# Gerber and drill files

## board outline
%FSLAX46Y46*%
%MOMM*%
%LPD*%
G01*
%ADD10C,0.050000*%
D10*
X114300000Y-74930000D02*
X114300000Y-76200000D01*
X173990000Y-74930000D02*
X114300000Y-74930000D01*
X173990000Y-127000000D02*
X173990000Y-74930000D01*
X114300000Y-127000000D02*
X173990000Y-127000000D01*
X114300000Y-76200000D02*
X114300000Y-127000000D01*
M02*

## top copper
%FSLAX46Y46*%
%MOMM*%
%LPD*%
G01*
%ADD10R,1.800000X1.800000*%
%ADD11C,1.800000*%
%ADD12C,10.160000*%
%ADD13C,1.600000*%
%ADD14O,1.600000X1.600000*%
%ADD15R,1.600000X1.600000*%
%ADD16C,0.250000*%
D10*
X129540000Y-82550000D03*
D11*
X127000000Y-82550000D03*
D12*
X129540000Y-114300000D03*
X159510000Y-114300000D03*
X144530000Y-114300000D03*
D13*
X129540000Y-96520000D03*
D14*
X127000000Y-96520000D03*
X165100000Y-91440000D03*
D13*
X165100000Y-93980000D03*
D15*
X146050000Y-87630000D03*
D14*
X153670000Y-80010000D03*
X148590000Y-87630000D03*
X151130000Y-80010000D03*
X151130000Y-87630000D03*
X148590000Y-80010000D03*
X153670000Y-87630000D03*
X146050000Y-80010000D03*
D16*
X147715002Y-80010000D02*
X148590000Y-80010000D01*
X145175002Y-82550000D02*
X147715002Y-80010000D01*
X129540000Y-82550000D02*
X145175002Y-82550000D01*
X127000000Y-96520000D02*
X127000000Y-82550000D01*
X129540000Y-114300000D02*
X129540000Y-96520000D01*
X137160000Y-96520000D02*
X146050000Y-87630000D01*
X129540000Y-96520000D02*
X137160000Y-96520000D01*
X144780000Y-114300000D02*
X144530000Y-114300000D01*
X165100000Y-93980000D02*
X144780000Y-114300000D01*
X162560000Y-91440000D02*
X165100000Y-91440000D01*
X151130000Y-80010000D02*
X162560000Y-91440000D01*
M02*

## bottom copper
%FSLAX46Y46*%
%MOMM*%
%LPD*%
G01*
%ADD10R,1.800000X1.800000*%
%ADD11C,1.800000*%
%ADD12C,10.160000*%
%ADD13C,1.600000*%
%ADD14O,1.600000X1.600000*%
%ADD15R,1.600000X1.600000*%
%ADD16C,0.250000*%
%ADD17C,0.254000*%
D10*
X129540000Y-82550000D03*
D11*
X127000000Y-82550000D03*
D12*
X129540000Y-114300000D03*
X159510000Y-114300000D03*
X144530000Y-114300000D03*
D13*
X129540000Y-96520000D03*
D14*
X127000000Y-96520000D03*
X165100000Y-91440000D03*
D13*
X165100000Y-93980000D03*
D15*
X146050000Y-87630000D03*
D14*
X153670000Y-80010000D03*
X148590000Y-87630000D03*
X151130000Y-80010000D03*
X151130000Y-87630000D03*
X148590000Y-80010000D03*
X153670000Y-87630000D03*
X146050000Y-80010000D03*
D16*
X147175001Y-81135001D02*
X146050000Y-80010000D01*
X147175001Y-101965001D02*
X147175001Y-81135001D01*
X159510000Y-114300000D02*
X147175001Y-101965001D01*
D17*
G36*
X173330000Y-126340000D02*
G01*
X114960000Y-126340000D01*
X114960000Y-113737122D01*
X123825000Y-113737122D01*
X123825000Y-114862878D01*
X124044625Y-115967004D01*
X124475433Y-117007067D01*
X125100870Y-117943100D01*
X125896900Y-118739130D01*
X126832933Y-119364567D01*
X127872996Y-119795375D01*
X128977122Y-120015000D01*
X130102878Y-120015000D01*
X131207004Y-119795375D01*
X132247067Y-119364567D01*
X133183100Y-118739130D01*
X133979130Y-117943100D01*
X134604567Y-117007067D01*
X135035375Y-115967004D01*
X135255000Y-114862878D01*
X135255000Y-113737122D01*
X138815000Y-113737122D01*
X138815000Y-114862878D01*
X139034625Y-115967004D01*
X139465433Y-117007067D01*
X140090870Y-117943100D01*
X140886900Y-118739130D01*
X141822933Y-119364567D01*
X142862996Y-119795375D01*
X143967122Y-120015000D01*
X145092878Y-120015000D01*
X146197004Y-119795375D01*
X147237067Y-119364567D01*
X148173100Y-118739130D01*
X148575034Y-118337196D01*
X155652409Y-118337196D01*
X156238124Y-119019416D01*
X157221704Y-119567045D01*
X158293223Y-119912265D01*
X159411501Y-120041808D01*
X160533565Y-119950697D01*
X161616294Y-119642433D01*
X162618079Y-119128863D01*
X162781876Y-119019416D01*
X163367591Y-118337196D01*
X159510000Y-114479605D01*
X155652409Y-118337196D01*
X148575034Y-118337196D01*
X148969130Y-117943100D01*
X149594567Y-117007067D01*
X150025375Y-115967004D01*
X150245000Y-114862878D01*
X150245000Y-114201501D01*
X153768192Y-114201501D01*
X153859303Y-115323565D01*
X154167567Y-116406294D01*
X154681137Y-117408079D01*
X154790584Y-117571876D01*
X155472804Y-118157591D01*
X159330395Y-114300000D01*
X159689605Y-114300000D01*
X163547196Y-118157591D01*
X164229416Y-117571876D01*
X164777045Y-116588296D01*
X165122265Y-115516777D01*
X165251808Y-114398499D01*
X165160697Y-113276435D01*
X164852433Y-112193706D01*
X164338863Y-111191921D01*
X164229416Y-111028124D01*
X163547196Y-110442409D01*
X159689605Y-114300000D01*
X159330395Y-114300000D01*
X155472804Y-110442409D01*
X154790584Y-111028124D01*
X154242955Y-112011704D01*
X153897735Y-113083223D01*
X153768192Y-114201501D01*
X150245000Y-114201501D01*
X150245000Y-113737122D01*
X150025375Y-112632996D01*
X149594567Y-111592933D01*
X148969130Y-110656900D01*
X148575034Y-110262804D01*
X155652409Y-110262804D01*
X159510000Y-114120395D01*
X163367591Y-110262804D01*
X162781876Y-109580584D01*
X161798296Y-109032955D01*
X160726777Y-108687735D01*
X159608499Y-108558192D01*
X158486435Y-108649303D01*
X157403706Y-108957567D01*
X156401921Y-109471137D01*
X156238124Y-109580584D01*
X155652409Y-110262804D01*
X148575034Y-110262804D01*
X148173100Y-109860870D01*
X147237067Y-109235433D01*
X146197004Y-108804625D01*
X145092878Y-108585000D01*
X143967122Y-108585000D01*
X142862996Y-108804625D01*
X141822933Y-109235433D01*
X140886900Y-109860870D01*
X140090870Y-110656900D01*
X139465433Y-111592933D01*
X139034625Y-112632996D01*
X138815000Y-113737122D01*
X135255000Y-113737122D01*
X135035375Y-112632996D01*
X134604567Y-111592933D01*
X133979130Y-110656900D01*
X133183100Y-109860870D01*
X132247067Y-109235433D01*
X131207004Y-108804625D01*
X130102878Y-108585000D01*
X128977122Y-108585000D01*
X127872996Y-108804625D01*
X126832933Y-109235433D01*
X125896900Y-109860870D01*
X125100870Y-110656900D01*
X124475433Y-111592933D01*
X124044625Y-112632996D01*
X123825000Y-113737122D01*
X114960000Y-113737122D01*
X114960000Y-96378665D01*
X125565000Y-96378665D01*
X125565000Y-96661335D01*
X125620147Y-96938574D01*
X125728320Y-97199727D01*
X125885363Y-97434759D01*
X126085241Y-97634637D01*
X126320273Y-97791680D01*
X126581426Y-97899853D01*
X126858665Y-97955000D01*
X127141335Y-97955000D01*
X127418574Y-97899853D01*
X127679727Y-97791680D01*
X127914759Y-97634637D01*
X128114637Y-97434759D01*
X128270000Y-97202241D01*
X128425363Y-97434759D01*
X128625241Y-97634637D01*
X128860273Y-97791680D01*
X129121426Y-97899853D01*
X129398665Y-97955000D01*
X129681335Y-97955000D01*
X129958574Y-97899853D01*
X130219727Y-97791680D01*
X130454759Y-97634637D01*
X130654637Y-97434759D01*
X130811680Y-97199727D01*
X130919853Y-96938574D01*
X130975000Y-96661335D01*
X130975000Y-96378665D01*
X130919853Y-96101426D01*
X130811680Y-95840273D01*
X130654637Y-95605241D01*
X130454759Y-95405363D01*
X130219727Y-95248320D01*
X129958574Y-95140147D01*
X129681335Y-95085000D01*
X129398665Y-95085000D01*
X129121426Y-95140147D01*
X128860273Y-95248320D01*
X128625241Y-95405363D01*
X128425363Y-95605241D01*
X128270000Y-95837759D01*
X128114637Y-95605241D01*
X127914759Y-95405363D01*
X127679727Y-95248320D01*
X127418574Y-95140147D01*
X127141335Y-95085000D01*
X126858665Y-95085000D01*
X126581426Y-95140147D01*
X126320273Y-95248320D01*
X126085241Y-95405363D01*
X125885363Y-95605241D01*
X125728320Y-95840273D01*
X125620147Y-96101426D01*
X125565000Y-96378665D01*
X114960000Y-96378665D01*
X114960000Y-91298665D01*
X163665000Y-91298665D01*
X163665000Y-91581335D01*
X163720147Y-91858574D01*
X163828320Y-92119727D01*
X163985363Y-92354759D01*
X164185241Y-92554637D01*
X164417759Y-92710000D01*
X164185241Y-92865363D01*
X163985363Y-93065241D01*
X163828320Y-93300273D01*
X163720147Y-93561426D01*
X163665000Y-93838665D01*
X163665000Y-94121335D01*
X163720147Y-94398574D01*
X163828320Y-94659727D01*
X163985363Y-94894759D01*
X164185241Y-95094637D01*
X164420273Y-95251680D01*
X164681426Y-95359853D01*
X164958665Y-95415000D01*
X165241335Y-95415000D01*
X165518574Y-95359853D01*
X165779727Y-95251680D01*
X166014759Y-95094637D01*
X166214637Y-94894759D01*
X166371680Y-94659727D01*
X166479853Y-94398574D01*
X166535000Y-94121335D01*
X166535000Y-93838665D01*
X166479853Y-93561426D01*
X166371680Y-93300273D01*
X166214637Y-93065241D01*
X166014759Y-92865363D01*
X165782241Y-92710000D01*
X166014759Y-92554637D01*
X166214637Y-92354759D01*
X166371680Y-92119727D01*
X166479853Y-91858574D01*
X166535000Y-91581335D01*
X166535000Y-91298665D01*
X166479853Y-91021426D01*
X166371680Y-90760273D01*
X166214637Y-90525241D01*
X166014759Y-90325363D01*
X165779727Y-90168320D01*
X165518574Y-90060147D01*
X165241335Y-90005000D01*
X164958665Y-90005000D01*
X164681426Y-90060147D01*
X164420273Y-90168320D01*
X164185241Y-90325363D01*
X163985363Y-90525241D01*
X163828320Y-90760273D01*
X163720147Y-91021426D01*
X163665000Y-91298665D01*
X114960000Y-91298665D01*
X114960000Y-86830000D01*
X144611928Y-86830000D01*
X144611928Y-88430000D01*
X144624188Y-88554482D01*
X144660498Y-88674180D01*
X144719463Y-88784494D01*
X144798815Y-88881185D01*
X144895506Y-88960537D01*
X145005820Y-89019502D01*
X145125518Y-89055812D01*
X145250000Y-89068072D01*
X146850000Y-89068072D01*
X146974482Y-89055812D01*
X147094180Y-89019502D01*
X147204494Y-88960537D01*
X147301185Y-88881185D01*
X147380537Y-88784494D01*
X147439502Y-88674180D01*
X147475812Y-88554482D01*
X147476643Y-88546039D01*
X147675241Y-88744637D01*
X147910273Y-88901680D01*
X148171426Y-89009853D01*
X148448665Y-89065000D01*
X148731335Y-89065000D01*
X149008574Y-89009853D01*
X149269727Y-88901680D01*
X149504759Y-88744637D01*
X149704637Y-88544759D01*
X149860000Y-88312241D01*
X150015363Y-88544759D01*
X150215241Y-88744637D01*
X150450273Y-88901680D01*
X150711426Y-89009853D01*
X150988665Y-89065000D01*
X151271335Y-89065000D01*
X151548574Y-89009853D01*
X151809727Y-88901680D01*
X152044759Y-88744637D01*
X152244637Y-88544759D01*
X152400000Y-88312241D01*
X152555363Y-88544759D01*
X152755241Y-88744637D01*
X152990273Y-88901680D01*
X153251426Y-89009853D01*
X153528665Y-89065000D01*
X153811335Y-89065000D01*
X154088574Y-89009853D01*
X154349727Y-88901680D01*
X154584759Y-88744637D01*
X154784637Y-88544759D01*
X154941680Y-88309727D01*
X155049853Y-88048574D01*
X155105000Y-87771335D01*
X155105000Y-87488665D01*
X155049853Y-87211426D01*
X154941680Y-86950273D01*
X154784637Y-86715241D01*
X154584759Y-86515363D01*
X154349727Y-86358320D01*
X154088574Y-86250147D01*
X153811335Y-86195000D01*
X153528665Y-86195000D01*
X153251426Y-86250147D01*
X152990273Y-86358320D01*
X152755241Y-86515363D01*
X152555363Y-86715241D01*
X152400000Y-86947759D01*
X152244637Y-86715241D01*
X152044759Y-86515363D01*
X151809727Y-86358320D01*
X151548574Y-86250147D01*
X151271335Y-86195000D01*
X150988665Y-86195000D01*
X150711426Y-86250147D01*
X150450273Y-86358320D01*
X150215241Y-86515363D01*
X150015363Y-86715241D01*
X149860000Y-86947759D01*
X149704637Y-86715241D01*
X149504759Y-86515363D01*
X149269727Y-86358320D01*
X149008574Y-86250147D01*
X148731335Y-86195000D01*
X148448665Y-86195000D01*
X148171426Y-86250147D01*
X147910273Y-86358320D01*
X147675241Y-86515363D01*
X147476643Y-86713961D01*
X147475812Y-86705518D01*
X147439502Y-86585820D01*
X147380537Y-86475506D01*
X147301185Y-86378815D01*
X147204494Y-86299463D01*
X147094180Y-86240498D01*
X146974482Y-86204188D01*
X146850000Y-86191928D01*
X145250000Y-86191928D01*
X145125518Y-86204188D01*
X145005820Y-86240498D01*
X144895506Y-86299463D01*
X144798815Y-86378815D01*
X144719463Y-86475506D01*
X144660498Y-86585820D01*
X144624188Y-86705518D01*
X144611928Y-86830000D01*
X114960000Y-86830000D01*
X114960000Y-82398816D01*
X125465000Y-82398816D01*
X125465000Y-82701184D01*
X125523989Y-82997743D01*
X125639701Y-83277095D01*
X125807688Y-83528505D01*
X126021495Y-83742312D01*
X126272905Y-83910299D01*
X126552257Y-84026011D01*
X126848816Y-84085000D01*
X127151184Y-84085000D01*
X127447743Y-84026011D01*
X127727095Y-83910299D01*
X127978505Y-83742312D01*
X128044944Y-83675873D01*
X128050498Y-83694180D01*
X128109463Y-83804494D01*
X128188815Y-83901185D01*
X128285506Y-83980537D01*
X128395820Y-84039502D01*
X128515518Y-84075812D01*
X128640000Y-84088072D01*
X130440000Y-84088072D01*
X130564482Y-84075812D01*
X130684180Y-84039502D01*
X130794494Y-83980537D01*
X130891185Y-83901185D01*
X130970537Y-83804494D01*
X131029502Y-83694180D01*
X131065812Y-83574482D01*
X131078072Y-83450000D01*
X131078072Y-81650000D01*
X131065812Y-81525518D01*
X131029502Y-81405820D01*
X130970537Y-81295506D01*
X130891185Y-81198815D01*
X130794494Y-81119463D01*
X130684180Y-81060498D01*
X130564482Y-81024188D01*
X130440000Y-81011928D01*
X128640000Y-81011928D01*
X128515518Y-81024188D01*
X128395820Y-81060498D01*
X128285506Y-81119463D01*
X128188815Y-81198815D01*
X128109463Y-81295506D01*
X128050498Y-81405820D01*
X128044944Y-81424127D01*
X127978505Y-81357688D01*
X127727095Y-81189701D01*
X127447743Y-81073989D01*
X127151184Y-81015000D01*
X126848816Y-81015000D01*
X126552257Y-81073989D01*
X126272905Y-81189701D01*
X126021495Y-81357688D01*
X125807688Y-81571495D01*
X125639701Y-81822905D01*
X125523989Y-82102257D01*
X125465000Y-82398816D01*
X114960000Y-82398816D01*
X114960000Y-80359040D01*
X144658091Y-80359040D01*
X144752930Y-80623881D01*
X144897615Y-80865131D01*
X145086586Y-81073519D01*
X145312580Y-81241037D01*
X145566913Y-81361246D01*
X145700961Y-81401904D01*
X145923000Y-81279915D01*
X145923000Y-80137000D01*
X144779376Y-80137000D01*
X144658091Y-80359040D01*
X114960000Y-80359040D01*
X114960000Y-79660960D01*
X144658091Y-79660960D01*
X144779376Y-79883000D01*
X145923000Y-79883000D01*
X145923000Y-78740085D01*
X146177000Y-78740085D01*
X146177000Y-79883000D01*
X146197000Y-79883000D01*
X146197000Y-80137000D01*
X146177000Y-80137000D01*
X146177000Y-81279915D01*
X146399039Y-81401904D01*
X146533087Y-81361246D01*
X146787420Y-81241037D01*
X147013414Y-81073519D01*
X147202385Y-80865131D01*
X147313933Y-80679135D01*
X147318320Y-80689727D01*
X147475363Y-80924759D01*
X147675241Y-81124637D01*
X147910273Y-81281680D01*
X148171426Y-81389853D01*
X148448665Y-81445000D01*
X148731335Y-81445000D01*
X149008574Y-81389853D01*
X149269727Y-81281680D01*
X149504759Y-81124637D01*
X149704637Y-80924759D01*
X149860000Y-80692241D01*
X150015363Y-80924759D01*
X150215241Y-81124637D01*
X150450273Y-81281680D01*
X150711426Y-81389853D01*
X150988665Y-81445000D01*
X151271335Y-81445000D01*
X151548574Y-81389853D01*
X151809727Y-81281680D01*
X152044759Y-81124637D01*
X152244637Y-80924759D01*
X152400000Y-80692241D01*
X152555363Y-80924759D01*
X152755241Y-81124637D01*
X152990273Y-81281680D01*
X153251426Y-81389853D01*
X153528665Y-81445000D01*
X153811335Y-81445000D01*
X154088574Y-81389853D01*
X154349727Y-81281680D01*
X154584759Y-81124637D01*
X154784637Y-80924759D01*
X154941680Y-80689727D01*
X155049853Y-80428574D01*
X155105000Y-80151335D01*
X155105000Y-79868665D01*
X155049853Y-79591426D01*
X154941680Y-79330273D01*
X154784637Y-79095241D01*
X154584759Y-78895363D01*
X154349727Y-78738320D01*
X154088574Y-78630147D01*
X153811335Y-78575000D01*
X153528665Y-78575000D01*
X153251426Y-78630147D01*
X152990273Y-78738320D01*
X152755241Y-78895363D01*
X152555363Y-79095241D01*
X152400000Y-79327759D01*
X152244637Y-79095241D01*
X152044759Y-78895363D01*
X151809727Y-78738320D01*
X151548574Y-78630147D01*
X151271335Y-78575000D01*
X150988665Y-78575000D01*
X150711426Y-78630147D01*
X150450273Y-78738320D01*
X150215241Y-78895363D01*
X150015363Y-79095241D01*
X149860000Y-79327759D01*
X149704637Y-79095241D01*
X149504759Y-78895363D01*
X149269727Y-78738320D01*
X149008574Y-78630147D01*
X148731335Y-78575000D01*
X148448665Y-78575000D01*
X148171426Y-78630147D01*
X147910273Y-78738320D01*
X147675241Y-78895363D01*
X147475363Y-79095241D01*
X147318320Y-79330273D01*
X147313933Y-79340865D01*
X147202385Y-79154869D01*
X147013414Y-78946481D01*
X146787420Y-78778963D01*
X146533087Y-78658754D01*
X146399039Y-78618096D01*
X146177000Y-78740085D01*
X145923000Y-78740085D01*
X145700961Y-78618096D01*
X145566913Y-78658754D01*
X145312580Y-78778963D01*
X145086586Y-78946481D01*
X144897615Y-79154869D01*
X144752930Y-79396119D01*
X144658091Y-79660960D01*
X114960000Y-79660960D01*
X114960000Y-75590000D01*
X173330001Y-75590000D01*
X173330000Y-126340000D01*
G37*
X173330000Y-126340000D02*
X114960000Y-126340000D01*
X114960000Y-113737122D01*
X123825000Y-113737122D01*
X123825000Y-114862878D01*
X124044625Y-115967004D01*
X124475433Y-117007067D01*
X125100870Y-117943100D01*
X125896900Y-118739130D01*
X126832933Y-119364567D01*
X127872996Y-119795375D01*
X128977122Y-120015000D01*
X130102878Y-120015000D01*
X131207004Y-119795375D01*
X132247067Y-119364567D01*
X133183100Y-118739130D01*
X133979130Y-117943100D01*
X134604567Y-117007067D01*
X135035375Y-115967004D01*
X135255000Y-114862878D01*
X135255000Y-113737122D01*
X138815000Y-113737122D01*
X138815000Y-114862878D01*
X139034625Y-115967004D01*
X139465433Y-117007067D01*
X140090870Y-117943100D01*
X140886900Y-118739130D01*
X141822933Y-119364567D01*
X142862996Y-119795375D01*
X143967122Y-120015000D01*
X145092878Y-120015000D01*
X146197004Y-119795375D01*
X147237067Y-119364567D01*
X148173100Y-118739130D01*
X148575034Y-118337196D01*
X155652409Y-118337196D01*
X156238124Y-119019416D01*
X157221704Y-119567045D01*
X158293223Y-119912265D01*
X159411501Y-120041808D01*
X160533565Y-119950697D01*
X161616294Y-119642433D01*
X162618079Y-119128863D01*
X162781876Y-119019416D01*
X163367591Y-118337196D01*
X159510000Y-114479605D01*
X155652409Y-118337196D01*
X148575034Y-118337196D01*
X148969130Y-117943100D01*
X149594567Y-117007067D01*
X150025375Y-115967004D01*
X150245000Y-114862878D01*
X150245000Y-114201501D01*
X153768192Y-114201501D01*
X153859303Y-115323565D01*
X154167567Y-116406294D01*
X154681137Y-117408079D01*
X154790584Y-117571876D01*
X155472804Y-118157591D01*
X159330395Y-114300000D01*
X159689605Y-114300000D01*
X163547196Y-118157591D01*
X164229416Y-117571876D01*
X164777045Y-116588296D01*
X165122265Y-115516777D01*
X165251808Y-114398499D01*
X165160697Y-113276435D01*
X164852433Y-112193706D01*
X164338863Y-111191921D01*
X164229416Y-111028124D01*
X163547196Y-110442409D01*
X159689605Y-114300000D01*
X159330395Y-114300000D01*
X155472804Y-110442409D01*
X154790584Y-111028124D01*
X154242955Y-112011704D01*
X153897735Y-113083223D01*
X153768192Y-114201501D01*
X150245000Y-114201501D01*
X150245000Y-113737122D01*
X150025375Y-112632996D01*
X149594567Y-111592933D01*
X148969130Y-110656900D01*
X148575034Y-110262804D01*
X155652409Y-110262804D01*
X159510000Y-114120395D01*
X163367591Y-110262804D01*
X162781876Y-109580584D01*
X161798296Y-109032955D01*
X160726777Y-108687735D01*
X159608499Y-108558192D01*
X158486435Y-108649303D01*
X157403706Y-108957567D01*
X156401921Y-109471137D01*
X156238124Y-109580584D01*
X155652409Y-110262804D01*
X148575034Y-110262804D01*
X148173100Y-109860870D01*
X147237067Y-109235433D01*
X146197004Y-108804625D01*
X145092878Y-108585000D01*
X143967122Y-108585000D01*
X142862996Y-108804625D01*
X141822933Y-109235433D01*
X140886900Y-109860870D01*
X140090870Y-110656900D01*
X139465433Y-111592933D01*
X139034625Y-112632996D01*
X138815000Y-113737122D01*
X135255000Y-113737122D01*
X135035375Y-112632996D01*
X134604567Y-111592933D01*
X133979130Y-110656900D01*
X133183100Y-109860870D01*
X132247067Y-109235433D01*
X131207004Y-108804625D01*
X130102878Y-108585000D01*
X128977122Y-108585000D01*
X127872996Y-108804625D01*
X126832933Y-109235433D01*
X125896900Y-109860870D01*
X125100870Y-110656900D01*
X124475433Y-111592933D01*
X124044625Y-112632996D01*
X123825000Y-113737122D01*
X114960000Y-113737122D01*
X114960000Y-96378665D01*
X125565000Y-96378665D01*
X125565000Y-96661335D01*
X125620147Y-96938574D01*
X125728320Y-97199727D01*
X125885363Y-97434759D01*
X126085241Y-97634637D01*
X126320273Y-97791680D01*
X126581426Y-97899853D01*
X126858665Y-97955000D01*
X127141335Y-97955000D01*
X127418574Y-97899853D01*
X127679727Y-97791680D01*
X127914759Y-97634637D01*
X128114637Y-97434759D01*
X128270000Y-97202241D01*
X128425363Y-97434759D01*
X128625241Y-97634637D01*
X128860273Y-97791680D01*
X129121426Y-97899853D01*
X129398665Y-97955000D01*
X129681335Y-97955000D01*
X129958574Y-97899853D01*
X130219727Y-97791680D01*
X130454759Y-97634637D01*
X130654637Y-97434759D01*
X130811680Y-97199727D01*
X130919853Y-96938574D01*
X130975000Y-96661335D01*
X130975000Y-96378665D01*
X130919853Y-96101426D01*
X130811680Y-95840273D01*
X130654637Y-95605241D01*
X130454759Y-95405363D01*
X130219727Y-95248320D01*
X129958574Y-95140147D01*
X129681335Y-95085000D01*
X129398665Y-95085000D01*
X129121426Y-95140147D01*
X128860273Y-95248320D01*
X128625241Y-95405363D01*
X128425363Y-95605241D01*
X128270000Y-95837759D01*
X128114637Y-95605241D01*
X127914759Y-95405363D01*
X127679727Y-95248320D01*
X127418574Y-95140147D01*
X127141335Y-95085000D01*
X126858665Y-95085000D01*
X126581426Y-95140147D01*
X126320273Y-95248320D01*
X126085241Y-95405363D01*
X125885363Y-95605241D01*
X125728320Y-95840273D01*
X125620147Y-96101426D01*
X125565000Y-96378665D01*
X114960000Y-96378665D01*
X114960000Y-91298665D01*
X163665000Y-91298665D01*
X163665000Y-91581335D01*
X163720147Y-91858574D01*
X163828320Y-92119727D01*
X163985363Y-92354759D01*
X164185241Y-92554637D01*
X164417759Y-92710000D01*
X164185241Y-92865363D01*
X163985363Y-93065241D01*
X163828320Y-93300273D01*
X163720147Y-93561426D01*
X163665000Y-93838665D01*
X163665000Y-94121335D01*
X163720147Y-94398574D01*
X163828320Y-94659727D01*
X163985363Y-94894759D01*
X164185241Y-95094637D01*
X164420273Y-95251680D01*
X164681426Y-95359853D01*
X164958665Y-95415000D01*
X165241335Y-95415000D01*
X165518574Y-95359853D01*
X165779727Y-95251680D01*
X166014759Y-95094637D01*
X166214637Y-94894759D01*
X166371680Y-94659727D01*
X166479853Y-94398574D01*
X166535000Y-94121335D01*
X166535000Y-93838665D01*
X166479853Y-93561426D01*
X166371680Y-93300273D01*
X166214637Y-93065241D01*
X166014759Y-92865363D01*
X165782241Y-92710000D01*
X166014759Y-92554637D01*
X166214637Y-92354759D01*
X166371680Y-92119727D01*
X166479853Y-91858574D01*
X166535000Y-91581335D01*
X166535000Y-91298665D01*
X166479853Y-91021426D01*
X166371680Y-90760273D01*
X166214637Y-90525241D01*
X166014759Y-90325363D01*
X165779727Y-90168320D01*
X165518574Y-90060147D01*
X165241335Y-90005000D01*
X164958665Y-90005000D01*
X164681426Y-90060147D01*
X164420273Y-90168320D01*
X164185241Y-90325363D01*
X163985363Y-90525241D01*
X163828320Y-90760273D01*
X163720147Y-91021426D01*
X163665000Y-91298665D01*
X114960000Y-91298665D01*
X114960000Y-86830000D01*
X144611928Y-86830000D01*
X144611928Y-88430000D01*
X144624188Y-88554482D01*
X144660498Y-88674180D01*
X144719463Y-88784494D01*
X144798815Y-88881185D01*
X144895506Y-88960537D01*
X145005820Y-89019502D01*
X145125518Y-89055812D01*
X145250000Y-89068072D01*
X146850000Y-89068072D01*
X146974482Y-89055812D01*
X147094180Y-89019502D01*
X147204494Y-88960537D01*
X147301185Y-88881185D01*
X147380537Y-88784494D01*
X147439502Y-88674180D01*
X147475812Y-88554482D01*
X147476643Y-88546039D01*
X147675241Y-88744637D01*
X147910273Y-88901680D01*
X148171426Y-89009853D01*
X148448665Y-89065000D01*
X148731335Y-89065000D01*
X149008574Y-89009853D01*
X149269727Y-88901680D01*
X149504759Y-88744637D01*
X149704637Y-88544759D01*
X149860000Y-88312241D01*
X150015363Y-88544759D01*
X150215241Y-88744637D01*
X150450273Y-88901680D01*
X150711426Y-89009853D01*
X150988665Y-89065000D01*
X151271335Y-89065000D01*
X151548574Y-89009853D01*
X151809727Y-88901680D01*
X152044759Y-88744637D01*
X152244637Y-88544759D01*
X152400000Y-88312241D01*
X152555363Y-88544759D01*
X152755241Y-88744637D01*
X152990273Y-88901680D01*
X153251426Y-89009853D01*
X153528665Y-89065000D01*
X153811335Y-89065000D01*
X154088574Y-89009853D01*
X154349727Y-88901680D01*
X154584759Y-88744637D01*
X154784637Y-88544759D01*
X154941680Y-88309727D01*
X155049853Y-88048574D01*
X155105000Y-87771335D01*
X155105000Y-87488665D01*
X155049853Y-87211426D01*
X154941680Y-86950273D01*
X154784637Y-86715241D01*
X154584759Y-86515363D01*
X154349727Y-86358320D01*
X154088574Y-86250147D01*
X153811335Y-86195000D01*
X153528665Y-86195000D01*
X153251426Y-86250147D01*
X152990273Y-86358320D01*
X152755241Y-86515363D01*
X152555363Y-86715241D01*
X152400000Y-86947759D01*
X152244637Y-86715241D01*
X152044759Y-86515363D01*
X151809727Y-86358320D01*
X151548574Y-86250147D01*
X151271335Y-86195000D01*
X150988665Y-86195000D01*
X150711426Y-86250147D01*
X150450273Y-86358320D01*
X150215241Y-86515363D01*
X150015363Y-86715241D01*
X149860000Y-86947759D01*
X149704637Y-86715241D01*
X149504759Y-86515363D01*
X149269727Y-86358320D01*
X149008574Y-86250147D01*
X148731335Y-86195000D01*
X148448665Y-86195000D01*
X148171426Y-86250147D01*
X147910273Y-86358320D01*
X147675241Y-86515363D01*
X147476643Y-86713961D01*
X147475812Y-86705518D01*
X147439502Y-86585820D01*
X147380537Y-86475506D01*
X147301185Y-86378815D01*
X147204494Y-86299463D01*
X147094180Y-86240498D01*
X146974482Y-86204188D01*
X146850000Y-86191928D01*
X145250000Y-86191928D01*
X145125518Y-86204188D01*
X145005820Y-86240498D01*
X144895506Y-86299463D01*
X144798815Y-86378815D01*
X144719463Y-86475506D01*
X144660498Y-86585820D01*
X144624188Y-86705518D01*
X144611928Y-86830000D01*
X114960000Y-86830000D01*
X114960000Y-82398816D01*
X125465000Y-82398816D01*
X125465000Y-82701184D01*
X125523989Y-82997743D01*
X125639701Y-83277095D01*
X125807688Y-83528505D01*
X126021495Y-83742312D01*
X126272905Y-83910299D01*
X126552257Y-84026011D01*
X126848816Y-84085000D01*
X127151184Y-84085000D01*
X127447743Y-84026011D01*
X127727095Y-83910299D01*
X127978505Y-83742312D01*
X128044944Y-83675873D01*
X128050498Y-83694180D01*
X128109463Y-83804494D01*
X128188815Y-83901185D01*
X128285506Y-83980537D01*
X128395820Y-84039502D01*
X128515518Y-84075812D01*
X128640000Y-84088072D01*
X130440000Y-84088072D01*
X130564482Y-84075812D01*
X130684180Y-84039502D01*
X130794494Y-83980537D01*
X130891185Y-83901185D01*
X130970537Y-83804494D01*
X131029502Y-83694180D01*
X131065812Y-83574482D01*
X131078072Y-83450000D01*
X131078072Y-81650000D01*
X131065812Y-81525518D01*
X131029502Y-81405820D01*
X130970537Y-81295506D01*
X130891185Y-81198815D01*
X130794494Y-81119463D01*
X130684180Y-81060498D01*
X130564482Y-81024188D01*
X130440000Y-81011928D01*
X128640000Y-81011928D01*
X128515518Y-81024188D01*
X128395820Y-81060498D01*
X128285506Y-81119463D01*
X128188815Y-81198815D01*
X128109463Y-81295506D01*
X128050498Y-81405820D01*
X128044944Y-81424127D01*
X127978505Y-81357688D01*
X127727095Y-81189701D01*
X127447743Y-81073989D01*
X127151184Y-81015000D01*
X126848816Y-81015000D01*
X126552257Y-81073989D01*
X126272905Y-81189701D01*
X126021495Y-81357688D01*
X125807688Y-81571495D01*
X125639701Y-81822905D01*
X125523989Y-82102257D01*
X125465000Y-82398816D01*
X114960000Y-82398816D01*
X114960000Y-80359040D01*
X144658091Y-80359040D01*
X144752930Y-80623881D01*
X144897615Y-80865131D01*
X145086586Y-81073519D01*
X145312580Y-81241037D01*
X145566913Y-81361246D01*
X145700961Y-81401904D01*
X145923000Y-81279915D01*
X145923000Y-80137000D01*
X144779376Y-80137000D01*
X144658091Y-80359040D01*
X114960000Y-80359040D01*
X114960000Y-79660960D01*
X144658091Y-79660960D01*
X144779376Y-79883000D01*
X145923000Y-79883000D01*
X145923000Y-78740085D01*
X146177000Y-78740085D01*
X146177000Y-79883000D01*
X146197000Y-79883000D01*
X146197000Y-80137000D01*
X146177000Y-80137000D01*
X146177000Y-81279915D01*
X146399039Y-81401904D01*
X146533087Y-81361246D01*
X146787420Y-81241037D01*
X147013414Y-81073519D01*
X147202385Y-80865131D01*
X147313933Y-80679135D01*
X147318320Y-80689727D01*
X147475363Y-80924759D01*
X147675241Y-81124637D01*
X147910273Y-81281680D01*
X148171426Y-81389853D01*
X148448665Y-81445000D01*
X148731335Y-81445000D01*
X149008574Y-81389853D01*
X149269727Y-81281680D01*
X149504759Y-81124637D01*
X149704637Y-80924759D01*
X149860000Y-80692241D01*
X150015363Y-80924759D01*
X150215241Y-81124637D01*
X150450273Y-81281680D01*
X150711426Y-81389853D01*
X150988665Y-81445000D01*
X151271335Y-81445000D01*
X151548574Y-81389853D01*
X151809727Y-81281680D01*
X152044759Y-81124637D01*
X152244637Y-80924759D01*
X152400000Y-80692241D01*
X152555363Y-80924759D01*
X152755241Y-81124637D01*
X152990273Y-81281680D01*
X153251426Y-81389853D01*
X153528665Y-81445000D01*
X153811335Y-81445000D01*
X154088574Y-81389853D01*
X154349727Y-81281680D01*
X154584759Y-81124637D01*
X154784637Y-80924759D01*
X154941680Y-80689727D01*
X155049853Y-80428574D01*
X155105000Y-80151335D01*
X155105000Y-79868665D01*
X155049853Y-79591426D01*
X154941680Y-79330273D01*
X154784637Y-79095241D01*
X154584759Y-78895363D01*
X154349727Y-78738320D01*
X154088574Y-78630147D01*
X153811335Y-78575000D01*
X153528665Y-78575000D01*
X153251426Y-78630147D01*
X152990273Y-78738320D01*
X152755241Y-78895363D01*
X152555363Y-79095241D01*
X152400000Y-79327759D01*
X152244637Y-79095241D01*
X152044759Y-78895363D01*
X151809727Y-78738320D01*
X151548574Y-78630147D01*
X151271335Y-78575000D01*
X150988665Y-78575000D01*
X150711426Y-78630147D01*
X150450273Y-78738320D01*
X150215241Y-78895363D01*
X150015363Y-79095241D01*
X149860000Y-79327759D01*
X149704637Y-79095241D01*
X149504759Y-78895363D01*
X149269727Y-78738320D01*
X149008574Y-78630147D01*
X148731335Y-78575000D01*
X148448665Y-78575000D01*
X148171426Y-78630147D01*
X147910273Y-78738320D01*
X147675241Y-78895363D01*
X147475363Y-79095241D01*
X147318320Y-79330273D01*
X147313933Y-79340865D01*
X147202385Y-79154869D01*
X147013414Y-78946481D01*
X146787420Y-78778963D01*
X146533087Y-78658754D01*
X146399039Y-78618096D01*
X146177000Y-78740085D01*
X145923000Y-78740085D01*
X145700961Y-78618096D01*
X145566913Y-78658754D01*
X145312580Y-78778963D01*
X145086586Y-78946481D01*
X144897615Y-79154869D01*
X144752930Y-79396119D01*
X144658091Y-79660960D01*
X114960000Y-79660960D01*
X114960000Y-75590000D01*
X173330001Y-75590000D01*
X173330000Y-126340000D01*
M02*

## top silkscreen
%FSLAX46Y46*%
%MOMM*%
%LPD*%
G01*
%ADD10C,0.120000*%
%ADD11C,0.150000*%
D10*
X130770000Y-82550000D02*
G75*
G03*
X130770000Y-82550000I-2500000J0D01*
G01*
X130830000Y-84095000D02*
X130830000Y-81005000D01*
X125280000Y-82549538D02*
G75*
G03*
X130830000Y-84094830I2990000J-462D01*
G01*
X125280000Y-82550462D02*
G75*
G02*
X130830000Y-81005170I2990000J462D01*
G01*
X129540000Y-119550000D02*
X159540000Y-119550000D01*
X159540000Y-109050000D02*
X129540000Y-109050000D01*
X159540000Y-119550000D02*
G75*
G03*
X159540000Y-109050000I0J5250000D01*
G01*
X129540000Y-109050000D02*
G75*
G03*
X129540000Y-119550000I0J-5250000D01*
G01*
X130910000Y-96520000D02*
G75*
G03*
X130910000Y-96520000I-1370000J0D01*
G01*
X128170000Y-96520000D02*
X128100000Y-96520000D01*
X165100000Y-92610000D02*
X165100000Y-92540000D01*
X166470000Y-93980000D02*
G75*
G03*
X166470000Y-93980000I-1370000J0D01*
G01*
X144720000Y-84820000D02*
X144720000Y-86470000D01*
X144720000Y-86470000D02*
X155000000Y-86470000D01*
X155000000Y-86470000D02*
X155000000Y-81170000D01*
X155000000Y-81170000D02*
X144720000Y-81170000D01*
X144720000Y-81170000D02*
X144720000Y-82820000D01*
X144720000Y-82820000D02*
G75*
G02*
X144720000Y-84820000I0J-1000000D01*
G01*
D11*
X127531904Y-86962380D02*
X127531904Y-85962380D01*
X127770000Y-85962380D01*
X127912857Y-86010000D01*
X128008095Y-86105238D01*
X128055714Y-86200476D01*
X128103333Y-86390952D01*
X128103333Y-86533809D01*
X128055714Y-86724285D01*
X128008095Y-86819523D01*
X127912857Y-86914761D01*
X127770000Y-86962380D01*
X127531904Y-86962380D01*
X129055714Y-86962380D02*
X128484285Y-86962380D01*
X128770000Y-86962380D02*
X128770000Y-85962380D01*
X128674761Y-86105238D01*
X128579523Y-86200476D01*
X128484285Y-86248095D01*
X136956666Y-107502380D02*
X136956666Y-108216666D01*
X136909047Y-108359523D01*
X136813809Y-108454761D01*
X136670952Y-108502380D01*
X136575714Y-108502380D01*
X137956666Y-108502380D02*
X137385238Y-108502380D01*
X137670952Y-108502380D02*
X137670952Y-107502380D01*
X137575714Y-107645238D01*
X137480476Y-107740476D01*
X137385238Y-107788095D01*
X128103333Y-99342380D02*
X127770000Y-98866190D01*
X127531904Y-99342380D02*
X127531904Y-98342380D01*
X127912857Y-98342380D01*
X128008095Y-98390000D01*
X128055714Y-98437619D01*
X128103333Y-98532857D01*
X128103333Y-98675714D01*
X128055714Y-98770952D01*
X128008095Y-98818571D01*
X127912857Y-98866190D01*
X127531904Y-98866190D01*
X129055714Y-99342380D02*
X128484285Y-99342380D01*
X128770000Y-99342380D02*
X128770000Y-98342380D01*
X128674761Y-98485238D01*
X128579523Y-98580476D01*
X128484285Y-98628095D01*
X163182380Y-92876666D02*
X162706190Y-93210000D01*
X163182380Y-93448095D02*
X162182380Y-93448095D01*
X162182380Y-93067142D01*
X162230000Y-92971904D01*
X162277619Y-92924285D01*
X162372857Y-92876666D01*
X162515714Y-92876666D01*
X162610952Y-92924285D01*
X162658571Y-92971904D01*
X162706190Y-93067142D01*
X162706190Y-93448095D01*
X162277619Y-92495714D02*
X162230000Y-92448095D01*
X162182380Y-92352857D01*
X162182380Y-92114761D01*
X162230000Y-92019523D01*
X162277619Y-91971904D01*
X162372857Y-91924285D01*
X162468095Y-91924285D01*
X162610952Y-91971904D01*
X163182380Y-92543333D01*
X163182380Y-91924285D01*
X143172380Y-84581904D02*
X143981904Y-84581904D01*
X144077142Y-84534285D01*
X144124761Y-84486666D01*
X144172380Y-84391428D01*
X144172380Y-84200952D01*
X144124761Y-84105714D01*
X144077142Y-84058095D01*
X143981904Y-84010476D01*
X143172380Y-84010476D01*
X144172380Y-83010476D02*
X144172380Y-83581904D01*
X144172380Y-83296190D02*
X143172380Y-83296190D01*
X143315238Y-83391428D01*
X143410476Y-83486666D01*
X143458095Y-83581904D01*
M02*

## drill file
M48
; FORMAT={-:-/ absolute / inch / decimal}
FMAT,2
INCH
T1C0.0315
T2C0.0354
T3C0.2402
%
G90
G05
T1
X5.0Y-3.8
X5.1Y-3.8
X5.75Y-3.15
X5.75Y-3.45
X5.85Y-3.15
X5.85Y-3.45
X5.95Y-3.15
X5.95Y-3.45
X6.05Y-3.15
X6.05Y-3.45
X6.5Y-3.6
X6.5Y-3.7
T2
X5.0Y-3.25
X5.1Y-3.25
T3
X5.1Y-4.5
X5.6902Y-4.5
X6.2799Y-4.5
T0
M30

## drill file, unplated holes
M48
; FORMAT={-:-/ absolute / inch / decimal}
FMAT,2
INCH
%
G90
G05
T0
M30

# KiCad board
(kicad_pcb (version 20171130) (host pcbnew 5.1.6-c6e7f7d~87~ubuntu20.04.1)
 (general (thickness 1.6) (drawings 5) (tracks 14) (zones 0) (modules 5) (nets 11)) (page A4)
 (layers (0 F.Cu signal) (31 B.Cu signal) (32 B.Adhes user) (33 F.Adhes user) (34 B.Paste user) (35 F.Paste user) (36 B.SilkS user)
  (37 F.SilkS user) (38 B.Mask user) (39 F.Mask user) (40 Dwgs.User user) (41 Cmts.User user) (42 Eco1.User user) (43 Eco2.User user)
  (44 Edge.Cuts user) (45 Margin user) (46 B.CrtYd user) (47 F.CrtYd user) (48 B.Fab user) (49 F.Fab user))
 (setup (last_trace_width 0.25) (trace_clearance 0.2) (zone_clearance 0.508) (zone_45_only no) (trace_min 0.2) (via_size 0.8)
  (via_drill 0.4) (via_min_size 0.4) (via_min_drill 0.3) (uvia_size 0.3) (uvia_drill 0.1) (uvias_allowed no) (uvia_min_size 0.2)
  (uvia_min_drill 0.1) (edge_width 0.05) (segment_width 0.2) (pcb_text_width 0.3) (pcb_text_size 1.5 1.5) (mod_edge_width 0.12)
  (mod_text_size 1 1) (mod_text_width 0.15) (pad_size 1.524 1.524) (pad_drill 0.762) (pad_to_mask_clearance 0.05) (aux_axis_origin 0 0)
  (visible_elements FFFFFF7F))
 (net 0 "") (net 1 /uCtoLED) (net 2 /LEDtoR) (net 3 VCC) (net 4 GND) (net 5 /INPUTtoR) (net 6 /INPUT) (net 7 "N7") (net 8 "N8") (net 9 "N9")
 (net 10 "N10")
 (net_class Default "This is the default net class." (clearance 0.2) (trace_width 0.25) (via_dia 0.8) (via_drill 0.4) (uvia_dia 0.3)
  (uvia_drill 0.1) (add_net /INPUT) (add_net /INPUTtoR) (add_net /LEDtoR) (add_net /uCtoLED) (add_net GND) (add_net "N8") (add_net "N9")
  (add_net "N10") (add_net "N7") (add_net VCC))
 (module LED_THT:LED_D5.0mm (layer F.Cu) (at 129.54 82.55 180)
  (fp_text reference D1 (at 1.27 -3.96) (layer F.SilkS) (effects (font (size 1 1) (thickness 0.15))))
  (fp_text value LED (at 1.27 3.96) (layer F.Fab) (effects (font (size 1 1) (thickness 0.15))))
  (fp_circle (center 1.27 0) (end 3.77 0) (layer F.SilkS) (width 0.12))
  (fp_line (start -1.29 -1.545) (end -1.29 1.545) (layer F.SilkS) (width 0.12))
  (fp_arc (start 1.27 0) (end -1.29 -1.54483) (angle 148.9) (layer F.SilkS) (width 0.12))
  (fp_arc (start 1.27 0) (end -1.29 1.54483) (angle -148.9) (layer F.SilkS) (width 0.12))
  (pad 1 thru_hole rect (at 0 0 180) (size 1.8 1.8) (drill 0.9) (layers *.Cu *.Mask) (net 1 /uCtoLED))
  (pad 2 thru_hole circle (at 2.54 0 180) (size 1.8 1.8) (drill 0.9) (layers *.Cu *.Mask) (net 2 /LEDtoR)))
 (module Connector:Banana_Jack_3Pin (layer F.Cu) (at 129.54 114.3)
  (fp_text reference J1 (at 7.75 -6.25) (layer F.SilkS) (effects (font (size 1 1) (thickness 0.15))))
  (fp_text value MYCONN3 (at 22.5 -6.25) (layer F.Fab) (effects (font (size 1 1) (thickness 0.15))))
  (fp_line (start 0 5.25) (end 30 5.25) (layer F.SilkS) (width 0.12))
  (fp_line (start 30 -5.25) (end 0 -5.25) (layer F.SilkS) (width 0.12))
  (fp_arc (start 30 0) (end 30 -5.25) (angle 180) (layer F.SilkS) (width 0.12))
  (fp_arc (start 0 0) (end 0 5.25) (angle 180) (layer F.SilkS) (width 0.12))
  (pad 1 thru_hole circle (at 0 0) (size 10.16 10.16) (drill 6.1) (layers *.Cu *.Mask) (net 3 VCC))
  (pad 3 thru_hole circle (at 29.97 0) (size 10.16 10.16) (drill 6.1) (layers *.Cu *.Mask) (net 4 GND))
  (pad 2 thru_hole circle (at 14.99 0) (size 10.16 10.16) (drill 6.1) (layers *.Cu *.Mask) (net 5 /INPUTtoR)))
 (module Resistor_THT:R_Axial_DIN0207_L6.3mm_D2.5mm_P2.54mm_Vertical (layer F.Cu) (at 129.54 96.52 180)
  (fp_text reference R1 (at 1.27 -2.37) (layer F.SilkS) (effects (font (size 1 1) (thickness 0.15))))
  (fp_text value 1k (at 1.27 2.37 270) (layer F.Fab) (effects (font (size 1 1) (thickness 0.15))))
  (fp_circle (center 0 0) (end 1.37 0) (layer F.SilkS) (width 0.12))
  (fp_line (start 1.37 0) (end 1.44 0) (layer F.SilkS) (width 0.12))
  (pad 1 thru_hole circle (at 0 0 180) (size 1.6 1.6) (drill 0.8) (layers *.Cu *.Mask) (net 3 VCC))
  (pad 2 thru_hole oval (at 2.54 0 180) (size 1.6 1.6) (drill 0.8) (layers *.Cu *.Mask) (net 2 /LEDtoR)))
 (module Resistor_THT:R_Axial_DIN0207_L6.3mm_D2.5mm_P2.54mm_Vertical (layer F.Cu) (at 165.1 93.98 90)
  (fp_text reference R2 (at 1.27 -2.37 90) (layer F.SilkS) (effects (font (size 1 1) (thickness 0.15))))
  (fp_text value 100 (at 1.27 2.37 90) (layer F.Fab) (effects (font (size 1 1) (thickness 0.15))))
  (fp_line (start 1.37 0) (end 1.44 0) (layer F.SilkS) (width 0.12))
  (fp_circle (center 0 0) (end 1.37 0) (layer F.SilkS) (width 0.12))
  (pad 2 thru_hole oval (at 2.54 0 90) (size 1.6 1.6) (drill 0.8) (layers *.Cu *.Mask) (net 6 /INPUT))
  (pad 1 thru_hole circle (at 0 0 90) (size 1.6 1.6) (drill 0.8) (layers *.Cu *.Mask) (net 5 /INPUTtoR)))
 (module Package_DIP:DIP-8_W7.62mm (layer F.Cu) (at 146.05 87.63 90)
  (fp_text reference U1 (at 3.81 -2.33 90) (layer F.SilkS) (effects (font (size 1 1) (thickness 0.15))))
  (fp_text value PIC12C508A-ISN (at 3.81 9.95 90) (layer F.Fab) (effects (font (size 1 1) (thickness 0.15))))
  (fp_line (start 2.81 -1.33) (end 1.16 -1.33) (layer F.SilkS) (width 0.12))
  (fp_line (start 1.16 -1.33) (end 1.16 8.95) (layer F.SilkS) (width 0.12))
  (fp_line (start 1.16 8.95) (end 6.46 8.95) (layer F.SilkS) (width 0.12))
  (fp_line (start 6.46 8.95) (end 6.46 -1.33) (layer F.SilkS) (width 0.12))
  (fp_line (start 6.46 -1.33) (end 4.81 -1.33) (layer F.SilkS) (width 0.12))
  (fp_arc (start 3.81 -1.33) (end 2.81 -1.33) (angle -180) (layer F.SilkS) (width 0.12))
  (pad 1 thru_hole rect (at 0 0 90) (size 1.6 1.6) (drill 0.8) (layers *.Cu *.Mask) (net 3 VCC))
  (pad 5 thru_hole oval (at 7.62 7.62 90) (size 1.6 1.6) (drill 0.8) (layers *.Cu *.Mask) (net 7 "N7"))
  (pad 2 thru_hole oval (at 0 2.54 90) (size 1.6 1.6) (drill 0.8) (layers *.Cu *.Mask) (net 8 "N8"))
  (pad 6 thru_hole oval (at 7.62 5.08 90) (size 1.6 1.6) (drill 0.8) (layers *.Cu *.Mask) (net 6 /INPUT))
  (pad 3 thru_hole oval (at 0 5.08 90) (size 1.6 1.6) (drill 0.8) (layers *.Cu *.Mask) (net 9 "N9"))
  (pad 7 thru_hole oval (at 7.62 2.54 90) (size 1.6 1.6) (drill 0.8) (layers *.Cu *.Mask) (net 1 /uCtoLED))
  (pad 4 thru_hole oval (at 0 7.62 90) (size 1.6 1.6) (drill 0.8) (layers *.Cu *.Mask) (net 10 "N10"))
  (pad 8 thru_hole oval (at 7.62 0 90) (size 1.6 1.6) (drill 0.8) (layers *.Cu *.Mask) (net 4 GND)))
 (gr_line (start 114.3 74.93) (end 114.3 76.2) (layer Edge.Cuts) (width 0.05))
 (gr_line (start 173.99 74.93) (end 114.3 74.93) (layer Edge.Cuts) (width 0.05))
 (gr_line (start 173.99 127) (end 173.99 74.93) (layer Edge.Cuts) (width 0.05))
 (gr_line (start 114.3 127) (end 173.99 127) (layer Edge.Cuts) (width 0.05))
 (gr_line (start 114.3 76.2) (end 114.3 127) (layer Edge.Cuts) (width 0.05))
 (segment (start 147.715002 80.01) (end 148.59 80.01) (width 0.25) (layer F.Cu) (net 1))
 (segment (start 145.175002 82.55) (end 147.715002 80.01) (width 0.25) (layer F.Cu) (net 1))
 (segment (start 129.54 82.55) (end 145.175002 82.55) (width 0.25) (layer F.Cu) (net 1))
 (segment (start 127 96.52) (end 127 82.55) (width 0.25) (layer F.Cu) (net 2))
 (segment (start 129.54 114.3) (end 129.54 96.52) (width 0.25) (layer F.Cu) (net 3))
 (segment (start 137.16 96.52) (end 146.05 87.63) (width 0.25) (layer F.Cu) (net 3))
 (segment (start 129.54 96.52) (end 137.16 96.52) (width 0.25) (layer F.Cu) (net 3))
 (segment (start 147.175001 81.135001) (end 146.05 80.01) (width 0.25) (layer B.Cu) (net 4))
 (segment (start 147.175001 101.965001) (end 147.175001 81.135001) (width 0.25) (layer B.Cu) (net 4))
 (segment (start 159.51 114.3) (end 147.175001 101.965001) (width 0.25) (layer B.Cu) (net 4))
 (segment (start 144.78 114.3) (end 144.53 114.3) (width 0.25) (layer F.Cu) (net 5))
 (segment (start 165.1 93.98) (end 144.78 114.3) (width 0.25) (layer F.Cu) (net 5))
 (segment (start 162.56 91.44) (end 165.1 91.44) (width 0.25) (layer F.Cu) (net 6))
 (segment (start 151.13 80.01) (end 162.56 91.44) (width 0.25) (layer F.Cu) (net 6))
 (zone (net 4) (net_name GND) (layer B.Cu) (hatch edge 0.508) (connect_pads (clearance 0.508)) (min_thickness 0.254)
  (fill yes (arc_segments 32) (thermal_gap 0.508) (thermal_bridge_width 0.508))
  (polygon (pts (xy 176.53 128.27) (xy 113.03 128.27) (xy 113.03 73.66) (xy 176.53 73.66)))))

